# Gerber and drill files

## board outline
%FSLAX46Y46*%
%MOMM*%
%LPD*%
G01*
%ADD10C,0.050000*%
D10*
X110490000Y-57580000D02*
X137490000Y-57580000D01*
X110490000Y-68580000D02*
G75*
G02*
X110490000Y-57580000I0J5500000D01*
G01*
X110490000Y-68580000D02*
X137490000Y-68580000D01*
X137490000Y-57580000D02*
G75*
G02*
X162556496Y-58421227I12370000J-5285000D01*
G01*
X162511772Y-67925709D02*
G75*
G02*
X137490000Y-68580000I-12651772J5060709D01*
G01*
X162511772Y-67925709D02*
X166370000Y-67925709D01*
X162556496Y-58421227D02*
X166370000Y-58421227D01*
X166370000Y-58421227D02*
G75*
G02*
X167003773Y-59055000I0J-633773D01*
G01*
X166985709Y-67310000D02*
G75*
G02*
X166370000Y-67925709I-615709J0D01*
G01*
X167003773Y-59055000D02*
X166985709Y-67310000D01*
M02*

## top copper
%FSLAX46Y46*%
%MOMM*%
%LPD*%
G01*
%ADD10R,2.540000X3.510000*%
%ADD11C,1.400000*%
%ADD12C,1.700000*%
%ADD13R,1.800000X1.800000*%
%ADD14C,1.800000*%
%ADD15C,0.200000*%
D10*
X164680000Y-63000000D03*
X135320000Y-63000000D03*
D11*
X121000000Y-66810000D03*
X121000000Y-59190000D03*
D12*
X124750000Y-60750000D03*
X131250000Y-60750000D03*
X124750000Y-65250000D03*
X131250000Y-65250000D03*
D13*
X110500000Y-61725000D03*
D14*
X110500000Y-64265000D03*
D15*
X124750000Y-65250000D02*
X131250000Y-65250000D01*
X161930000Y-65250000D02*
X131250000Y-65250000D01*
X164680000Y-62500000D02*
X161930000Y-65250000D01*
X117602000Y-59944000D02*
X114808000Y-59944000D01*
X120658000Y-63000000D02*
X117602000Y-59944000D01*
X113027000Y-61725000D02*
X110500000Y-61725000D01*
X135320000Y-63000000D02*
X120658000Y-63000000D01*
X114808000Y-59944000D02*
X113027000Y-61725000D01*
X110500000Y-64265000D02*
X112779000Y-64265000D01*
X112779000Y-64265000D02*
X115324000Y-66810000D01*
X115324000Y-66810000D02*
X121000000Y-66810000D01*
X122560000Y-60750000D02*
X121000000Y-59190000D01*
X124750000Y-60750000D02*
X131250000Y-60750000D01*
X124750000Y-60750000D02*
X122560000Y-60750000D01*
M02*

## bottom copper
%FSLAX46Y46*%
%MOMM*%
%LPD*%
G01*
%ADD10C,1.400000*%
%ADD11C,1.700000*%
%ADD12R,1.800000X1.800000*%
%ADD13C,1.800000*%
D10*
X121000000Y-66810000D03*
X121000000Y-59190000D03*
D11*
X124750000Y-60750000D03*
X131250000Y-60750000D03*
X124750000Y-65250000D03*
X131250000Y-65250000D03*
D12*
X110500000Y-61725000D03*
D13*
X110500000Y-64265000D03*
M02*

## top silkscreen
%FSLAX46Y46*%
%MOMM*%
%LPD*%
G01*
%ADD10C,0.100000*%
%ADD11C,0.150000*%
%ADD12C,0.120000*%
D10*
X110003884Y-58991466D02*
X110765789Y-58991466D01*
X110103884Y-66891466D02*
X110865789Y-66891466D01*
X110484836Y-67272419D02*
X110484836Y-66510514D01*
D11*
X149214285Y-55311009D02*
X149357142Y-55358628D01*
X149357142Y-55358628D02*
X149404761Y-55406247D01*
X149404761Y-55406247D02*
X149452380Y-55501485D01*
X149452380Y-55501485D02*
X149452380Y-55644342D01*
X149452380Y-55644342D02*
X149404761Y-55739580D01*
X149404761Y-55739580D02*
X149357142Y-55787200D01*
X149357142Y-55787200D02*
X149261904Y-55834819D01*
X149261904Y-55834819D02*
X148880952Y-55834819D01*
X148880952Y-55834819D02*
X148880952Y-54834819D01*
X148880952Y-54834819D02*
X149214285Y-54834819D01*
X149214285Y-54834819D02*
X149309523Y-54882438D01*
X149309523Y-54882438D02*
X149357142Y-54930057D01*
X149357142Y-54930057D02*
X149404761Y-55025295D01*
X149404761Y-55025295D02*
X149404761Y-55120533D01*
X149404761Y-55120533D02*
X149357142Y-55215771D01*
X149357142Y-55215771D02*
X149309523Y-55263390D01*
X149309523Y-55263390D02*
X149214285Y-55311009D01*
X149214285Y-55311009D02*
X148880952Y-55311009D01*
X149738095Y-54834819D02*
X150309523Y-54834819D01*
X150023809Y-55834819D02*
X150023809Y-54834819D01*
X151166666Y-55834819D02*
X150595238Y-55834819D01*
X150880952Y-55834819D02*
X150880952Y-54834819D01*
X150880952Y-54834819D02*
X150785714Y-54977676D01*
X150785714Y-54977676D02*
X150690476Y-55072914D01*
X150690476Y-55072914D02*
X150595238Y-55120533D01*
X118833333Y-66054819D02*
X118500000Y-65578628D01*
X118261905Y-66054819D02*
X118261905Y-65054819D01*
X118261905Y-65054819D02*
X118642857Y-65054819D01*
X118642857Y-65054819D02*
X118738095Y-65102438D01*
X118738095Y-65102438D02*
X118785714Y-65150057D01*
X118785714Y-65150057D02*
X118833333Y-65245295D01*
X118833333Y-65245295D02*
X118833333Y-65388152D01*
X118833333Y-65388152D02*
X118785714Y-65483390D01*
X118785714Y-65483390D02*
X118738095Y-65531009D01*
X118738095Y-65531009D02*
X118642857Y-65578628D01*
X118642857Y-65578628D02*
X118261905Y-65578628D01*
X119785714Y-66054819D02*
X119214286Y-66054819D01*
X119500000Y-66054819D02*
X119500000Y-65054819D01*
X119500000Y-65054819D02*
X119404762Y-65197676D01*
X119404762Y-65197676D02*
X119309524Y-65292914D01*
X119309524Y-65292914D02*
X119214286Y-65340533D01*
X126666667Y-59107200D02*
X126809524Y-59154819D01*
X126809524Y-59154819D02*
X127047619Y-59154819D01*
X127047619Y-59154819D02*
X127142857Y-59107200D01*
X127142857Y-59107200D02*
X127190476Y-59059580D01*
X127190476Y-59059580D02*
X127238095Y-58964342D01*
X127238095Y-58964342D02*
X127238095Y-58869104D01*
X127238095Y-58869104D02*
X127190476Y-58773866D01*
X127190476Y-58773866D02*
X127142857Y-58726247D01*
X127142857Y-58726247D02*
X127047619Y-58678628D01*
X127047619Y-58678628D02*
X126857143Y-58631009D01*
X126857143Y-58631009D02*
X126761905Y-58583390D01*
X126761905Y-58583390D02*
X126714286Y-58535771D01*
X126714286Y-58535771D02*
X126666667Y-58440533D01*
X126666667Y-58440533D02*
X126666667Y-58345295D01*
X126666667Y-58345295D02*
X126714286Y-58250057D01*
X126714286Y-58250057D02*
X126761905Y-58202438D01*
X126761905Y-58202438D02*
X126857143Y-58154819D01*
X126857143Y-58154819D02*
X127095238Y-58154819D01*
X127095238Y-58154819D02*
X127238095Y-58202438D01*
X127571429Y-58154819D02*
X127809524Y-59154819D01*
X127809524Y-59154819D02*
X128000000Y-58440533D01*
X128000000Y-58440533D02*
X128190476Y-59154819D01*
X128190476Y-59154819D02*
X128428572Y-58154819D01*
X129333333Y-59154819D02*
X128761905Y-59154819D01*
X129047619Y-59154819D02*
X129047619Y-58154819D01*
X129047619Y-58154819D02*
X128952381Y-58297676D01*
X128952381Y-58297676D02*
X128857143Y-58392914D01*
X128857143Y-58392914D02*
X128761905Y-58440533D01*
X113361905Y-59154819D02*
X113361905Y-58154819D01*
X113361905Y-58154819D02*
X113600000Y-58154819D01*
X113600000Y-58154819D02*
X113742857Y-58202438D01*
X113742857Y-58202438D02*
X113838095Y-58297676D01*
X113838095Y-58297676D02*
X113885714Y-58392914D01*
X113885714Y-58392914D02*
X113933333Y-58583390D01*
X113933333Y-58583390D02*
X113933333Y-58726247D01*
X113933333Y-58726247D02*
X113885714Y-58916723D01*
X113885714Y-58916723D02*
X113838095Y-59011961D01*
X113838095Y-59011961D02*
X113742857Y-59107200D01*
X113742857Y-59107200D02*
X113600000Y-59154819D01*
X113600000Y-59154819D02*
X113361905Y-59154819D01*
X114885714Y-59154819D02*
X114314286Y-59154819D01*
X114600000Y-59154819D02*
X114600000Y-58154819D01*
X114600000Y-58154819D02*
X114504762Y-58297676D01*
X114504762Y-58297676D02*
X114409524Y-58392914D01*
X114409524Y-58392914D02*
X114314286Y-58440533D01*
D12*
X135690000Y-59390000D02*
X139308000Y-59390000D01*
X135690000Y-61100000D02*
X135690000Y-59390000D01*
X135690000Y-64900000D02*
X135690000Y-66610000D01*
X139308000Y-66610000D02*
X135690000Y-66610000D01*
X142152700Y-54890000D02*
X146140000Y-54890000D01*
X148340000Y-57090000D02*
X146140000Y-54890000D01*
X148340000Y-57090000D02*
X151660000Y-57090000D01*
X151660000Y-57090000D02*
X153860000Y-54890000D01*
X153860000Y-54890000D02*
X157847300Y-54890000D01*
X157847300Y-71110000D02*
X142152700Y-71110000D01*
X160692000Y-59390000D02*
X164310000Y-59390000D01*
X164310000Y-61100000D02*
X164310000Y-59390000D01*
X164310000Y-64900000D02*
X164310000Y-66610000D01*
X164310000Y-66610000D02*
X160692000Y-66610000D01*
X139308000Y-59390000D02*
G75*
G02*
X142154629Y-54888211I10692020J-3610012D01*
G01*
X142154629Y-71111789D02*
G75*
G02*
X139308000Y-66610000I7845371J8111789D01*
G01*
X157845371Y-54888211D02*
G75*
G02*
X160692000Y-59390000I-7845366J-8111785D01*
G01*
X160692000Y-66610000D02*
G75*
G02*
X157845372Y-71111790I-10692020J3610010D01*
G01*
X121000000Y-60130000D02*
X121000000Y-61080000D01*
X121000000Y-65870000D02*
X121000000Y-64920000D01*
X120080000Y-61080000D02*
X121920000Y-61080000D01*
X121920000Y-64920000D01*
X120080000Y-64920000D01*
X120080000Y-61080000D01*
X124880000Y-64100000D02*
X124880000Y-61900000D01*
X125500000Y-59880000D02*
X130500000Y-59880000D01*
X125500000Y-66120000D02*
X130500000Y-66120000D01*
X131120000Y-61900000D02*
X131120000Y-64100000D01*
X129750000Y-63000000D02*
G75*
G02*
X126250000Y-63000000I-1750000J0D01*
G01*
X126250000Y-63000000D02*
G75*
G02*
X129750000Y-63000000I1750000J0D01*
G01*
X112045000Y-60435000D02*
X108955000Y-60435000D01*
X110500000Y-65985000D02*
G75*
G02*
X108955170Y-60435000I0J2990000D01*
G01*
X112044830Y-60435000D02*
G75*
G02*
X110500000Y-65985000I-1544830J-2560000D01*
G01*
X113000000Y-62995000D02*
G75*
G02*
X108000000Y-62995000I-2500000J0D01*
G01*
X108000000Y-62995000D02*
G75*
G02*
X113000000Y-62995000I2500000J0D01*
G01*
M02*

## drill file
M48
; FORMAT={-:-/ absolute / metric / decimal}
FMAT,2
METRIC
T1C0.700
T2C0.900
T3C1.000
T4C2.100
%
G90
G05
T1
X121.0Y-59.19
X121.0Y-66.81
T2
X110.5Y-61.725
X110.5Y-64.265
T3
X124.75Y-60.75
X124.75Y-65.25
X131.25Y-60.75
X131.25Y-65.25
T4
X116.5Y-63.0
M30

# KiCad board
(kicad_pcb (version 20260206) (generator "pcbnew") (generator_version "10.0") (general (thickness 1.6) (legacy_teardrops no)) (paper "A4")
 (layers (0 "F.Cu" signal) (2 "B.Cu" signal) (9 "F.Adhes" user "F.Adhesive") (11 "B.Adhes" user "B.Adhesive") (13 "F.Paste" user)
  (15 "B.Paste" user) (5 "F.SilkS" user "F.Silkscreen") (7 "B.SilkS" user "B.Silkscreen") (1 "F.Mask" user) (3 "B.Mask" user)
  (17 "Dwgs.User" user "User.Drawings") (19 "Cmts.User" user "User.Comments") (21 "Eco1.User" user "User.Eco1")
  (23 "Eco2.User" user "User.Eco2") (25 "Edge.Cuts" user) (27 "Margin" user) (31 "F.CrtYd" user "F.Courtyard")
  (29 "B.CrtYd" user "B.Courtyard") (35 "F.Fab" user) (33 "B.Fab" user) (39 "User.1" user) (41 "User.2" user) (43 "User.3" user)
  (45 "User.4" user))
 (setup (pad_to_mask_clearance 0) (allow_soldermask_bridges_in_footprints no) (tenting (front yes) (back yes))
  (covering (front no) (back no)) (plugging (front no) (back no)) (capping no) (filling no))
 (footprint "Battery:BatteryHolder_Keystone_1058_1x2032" (layer "F.Cu") (at 150 63 180)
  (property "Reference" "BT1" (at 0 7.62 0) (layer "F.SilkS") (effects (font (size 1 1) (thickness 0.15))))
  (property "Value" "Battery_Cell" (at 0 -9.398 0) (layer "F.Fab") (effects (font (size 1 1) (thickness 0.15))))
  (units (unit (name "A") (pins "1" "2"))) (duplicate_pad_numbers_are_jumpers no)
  (fp_line (start 14.31 3.61) (end 10.692 3.61) (stroke (width 0.12) (type solid)) (layer "F.SilkS"))
  (fp_line (start 14.31 1.9) (end 14.31 3.61) (stroke (width 0.12) (type solid)) (layer "F.SilkS"))
  (fp_line (start 14.31 -1.9) (end 14.31 -3.61) (stroke (width 0.12) (type solid)) (layer "F.SilkS"))
  (fp_line (start 10.692 -3.61) (end 14.31 -3.61) (stroke (width 0.12) (type solid)) (layer "F.SilkS"))
  (fp_line (start 7.8473 8.11) (end 3.86 8.11) (stroke (width 0.12) (type solid)) (layer "F.SilkS"))
  (fp_line (start 1.66 5.91) (end 3.86 8.11) (stroke (width 0.12) (type solid)) (layer "F.SilkS"))
  (fp_line (start 1.66 5.91) (end -1.66 5.91) (stroke (width 0.12) (type solid)) (layer "F.SilkS"))
  (fp_line (start -1.66 5.91) (end -3.86 8.11) (stroke (width 0.12) (type solid)) (layer "F.SilkS"))
  (fp_line (start -3.86 8.11) (end -7.8473 8.11) (stroke (width 0.12) (type solid)) (layer "F.SilkS"))
  (fp_line (start -7.8473 -8.11) (end 7.8473 -8.11) (stroke (width 0.12) (type solid)) (layer "F.SilkS"))
  (fp_line (start -10.692 3.61) (end -14.31 3.61) (stroke (width 0.12) (type solid)) (layer "F.SilkS"))
  (fp_line (start -14.31 1.9) (end -14.31 3.61) (stroke (width 0.12) (type solid)) (layer "F.SilkS"))
  (fp_line (start -14.31 -1.9) (end -14.31 -3.61) (stroke (width 0.12) (type solid)) (layer "F.SilkS"))
  (fp_line (start -14.31 -3.61) (end -10.692 -3.61) (stroke (width 0.12) (type solid)) (layer "F.SilkS"))
  (fp_arc (start 10.692 3.61) (mid 9.538084 6.031244) (end 7.845371 8.111789) (stroke (width 0.12) (type solid)) (layer "F.SilkS"))
  (fp_arc (start 7.845371 -8.111789) (mid 9.538085 -6.031244) (end 10.692 -3.61) (stroke (width 0.12) (type solid)) (layer "F.SilkS"))
  (fp_arc (start -7.845371 8.111789) (mid -9.538085 6.031244) (end -10.692 3.61) (stroke (width 0.12) (type solid)) (layer "F.SilkS"))
  (fp_arc (start -10.692 -3.61) (mid -9.538084 -6.031244) (end -7.845371 -8.111789) (stroke (width 0.12) (type solid)) (layer "F.SilkS"))
  (pad "1" smd rect (at -14.68 0 180) (size 2.54 3.51) (layers "F.Cu" "F.Mask" "F.Paste") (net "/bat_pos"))
  (pad "2" smd rect (at 14.68 0 180) (size 2.54 3.51) (layers "F.Cu" "F.Mask" "F.Paste") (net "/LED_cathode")))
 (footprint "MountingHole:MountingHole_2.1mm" (layer "F.Cu") (at 116.5 63)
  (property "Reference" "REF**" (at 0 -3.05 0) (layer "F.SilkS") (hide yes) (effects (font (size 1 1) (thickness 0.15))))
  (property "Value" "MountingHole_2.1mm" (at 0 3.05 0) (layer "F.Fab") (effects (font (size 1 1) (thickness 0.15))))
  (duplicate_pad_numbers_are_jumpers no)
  (pad "" np_thru_hole circle (at 0 0) (size 2.1 2.1) (drill 2.1) (layers "*.Cu" "*.Mask")))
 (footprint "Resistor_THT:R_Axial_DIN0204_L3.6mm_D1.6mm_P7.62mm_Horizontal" (layer "F.Cu") (at 121 66.81 90)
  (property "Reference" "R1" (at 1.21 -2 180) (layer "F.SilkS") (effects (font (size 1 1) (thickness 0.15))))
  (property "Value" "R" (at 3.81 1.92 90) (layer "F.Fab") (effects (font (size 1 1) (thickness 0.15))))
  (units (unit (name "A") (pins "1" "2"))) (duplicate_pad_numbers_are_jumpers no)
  (fp_line (start 6.68 0) (end 5.73 0) (stroke (width 0.12) (type solid)) (layer "F.SilkS"))
  (fp_line (start 0.94 0) (end 1.89 0) (stroke (width 0.12) (type solid)) (layer "F.SilkS"))
  (fp_rect (start 1.89 -0.92) (end 5.73 0.92) (stroke (width 0.12) (type solid)) (fill no) (layer "F.SilkS"))
  (pad "1" thru_hole circle (at 0 0 90) (size 1.4 1.4) (drill 0.7) (layers "*.Cu" "*.Mask") (remove_unused_layers no) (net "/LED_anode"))
  (pad "2" thru_hole circle (at 7.62 0 90) (size 1.4 1.4) (drill 0.7) (layers "*.Cu" "*.Mask") (remove_unused_layers no)
   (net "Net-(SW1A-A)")))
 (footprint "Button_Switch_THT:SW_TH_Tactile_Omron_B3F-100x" (layer "F.Cu") (at 124.75 60.75)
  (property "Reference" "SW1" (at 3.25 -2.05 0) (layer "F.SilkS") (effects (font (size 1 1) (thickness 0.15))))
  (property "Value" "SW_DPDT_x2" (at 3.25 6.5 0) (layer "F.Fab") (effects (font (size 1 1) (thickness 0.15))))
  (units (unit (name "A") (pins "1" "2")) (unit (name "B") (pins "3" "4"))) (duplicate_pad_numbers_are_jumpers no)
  (fp_line (start 0.13 3.35) (end 0.13 1.15) (stroke (width 0.12) (type solid)) (layer "F.SilkS"))
  (fp_line (start 0.75 -0.87) (end 5.75 -0.87) (stroke (width 0.12) (type solid)) (layer "F.SilkS"))
  (fp_line (start 0.75 5.37) (end 5.75 5.37) (stroke (width 0.12) (type solid)) (layer "F.SilkS"))
  (fp_line (start 6.37 1.15) (end 6.37 3.35) (stroke (width 0.12) (type solid)) (layer "F.SilkS"))
  (fp_circle (center 3.25 2.25) (end 5 2.25) (stroke (width 0.12) (type solid)) (fill no) (layer "F.SilkS"))
  (pad "1" thru_hole circle (at 0 0) (size 1.7 1.7) (drill 1) (layers "*.Cu" "*.Mask") (remove_unused_layers no) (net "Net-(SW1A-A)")
   (thermal_bridge_angle 90))
  (pad "1" thru_hole circle (at 6.5 0) (size 1.7 1.7) (drill 1) (layers "*.Cu" "*.Mask") (remove_unused_layers no) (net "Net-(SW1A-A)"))
  (pad "2" thru_hole circle (at 0 4.5) (size 1.7 1.7) (drill 1) (layers "*.Cu" "*.Mask") (remove_unused_layers no) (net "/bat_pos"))
  (pad "2" thru_hole circle (at 6.5 4.5) (size 1.7 1.7) (drill 1) (layers "*.Cu" "*.Mask") (remove_unused_layers no) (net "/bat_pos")))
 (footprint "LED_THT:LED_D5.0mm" (layer "F.Cu") (at 110.5 61.725 -90)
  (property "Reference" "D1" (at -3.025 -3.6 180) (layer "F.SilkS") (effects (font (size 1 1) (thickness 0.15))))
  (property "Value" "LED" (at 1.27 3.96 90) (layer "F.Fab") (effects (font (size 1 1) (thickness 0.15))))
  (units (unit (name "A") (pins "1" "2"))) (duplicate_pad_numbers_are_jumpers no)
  (fp_line (start -1.29 -1.545) (end -1.29 1.545) (stroke (width 0.12) (type solid)) (layer "F.SilkS"))
  (fp_arc (start 4.26 0) (mid 2.071779 2.880495) (end -1.29 1.54483) (stroke (width 0.12) (type solid)) (layer "F.SilkS"))
  (fp_arc (start -1.29 -1.54483) (mid 2.071779 -2.880495) (end 4.26 0) (stroke (width 0.12) (type solid)) (layer "F.SilkS"))
  (fp_circle (center 1.27 0) (end 3.77 0) (stroke (width 0.12) (type solid)) (fill no) (layer "F.SilkS"))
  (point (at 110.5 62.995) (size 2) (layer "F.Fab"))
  (pad "1" thru_hole rect (at 0 0 270) (size 1.8 1.8) (drill 0.9) (layers "*.Cu" "*.Mask") (remove_unused_layers no) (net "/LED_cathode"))
  (pad "2" thru_hole circle (at 2.54 0 270) (size 1.8 1.8) (drill 0.9) (layers "*.Cu" "*.Mask") (remove_unused_layers no) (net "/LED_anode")))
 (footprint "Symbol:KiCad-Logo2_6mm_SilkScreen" (layer "B.Cu") (at 150 62.5 180)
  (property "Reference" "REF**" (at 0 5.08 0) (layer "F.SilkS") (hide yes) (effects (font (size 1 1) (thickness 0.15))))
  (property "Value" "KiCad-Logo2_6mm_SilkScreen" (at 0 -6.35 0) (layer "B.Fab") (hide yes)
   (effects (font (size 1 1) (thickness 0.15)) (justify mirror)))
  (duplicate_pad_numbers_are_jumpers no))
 (gr_line (start 110.49 57.58) (end 137.49 57.58) (stroke (width 0.05) (type default)) (layer "Edge.Cuts"))
 (gr_arc (start 110.49 68.58) (mid 104.99 63.08) (end 110.49 57.58) (stroke (width 0.05) (type default)) (layer "Edge.Cuts"))
 (gr_line (start 110.49 68.58) (end 137.49 68.58) (stroke (width 0.05) (type default)) (layer "Edge.Cuts"))
 (gr_arc (start 137.49 57.58) (mid 150.311182 49.420873) (end 162.556496 58.421227) (stroke (width 0.05) (type default)) (layer "Edge.Cuts"))
 (gr_arc (start 162.511772 67.925709) (mid 150.216192 76.486719) (end 137.49 68.58) (stroke (width 0.05) (type default)) (layer "Edge.Cuts"))
 (gr_line (start 162.511772 67.925709) (end 166.37 67.925709) (stroke (width 0.05) (type default)) (layer "Edge.Cuts"))
 (gr_line (start 162.556496 58.421227) (end 166.37 58.421227) (stroke (width 0.05) (type default)) (layer "Edge.Cuts"))
 (gr_arc (start 166.37 58.421227) (mid 166.818145 58.606855) (end 167.003773 59.055) (stroke (width 0.05) (type default))
  (layer "Edge.Cuts"))
 (gr_arc (start 166.985709 67.31) (mid 166.805372 67.745372) (end 166.37 67.925709) (stroke (width 0.05) (type default)) (layer "Edge.Cuts"))
 (gr_line (start 167.003773 59.055) (end 166.985709 67.31) (stroke (width 0.05) (type default)) (layer "Edge.Cuts"))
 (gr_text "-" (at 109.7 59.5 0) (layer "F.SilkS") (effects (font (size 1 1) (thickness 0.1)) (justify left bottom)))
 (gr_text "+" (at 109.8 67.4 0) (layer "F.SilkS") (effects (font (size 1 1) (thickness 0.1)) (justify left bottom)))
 (segment (start 124.75 65.25) (end 131.25 65.25) (width 0.2) (layer "F.Cu") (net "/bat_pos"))
 (segment (start 161.93 65.25) (end 131.25 65.25) (width 0.2) (layer "F.Cu") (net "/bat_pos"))
 (segment (start 164.68 62.5) (end 161.93 65.25) (width 0.2) (layer "F.Cu") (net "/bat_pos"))
 (segment (start 117.602 59.944) (end 114.808 59.944) (width 0.2) (layer "F.Cu") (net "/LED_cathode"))
 (segment (start 120.658 63) (end 117.602 59.944) (width 0.2) (layer "F.Cu") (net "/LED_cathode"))
 (segment (start 113.027 61.725) (end 110.5 61.725) (width 0.2) (layer "F.Cu") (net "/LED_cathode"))
 (segment (start 135.32 63) (end 120.658 63) (width 0.2) (layer "F.Cu") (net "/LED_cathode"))
 (segment (start 114.808 59.944) (end 113.027 61.725) (width 0.2) (layer "F.Cu") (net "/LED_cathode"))
 (segment (start 110.5 64.265) (end 112.779 64.265) (width 0.2) (layer "F.Cu") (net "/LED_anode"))
 (segment (start 112.779 64.265) (end 115.324 66.81) (width 0.2) (layer "F.Cu") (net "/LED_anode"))
 (segment (start 115.324 66.81) (end 121 66.81) (width 0.2) (layer "F.Cu") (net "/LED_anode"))
 (segment (start 122.56 60.75) (end 121 59.19) (width 0.2) (layer "F.Cu") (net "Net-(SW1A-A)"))
 (segment (start 124.75 60.75) (end 131.25 60.75) (width 0.2) (layer "F.Cu") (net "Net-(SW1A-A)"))
 (segment (start 124.75 60.75) (end 122.56 60.75) (width 0.2) (layer "F.Cu") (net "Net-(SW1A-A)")))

